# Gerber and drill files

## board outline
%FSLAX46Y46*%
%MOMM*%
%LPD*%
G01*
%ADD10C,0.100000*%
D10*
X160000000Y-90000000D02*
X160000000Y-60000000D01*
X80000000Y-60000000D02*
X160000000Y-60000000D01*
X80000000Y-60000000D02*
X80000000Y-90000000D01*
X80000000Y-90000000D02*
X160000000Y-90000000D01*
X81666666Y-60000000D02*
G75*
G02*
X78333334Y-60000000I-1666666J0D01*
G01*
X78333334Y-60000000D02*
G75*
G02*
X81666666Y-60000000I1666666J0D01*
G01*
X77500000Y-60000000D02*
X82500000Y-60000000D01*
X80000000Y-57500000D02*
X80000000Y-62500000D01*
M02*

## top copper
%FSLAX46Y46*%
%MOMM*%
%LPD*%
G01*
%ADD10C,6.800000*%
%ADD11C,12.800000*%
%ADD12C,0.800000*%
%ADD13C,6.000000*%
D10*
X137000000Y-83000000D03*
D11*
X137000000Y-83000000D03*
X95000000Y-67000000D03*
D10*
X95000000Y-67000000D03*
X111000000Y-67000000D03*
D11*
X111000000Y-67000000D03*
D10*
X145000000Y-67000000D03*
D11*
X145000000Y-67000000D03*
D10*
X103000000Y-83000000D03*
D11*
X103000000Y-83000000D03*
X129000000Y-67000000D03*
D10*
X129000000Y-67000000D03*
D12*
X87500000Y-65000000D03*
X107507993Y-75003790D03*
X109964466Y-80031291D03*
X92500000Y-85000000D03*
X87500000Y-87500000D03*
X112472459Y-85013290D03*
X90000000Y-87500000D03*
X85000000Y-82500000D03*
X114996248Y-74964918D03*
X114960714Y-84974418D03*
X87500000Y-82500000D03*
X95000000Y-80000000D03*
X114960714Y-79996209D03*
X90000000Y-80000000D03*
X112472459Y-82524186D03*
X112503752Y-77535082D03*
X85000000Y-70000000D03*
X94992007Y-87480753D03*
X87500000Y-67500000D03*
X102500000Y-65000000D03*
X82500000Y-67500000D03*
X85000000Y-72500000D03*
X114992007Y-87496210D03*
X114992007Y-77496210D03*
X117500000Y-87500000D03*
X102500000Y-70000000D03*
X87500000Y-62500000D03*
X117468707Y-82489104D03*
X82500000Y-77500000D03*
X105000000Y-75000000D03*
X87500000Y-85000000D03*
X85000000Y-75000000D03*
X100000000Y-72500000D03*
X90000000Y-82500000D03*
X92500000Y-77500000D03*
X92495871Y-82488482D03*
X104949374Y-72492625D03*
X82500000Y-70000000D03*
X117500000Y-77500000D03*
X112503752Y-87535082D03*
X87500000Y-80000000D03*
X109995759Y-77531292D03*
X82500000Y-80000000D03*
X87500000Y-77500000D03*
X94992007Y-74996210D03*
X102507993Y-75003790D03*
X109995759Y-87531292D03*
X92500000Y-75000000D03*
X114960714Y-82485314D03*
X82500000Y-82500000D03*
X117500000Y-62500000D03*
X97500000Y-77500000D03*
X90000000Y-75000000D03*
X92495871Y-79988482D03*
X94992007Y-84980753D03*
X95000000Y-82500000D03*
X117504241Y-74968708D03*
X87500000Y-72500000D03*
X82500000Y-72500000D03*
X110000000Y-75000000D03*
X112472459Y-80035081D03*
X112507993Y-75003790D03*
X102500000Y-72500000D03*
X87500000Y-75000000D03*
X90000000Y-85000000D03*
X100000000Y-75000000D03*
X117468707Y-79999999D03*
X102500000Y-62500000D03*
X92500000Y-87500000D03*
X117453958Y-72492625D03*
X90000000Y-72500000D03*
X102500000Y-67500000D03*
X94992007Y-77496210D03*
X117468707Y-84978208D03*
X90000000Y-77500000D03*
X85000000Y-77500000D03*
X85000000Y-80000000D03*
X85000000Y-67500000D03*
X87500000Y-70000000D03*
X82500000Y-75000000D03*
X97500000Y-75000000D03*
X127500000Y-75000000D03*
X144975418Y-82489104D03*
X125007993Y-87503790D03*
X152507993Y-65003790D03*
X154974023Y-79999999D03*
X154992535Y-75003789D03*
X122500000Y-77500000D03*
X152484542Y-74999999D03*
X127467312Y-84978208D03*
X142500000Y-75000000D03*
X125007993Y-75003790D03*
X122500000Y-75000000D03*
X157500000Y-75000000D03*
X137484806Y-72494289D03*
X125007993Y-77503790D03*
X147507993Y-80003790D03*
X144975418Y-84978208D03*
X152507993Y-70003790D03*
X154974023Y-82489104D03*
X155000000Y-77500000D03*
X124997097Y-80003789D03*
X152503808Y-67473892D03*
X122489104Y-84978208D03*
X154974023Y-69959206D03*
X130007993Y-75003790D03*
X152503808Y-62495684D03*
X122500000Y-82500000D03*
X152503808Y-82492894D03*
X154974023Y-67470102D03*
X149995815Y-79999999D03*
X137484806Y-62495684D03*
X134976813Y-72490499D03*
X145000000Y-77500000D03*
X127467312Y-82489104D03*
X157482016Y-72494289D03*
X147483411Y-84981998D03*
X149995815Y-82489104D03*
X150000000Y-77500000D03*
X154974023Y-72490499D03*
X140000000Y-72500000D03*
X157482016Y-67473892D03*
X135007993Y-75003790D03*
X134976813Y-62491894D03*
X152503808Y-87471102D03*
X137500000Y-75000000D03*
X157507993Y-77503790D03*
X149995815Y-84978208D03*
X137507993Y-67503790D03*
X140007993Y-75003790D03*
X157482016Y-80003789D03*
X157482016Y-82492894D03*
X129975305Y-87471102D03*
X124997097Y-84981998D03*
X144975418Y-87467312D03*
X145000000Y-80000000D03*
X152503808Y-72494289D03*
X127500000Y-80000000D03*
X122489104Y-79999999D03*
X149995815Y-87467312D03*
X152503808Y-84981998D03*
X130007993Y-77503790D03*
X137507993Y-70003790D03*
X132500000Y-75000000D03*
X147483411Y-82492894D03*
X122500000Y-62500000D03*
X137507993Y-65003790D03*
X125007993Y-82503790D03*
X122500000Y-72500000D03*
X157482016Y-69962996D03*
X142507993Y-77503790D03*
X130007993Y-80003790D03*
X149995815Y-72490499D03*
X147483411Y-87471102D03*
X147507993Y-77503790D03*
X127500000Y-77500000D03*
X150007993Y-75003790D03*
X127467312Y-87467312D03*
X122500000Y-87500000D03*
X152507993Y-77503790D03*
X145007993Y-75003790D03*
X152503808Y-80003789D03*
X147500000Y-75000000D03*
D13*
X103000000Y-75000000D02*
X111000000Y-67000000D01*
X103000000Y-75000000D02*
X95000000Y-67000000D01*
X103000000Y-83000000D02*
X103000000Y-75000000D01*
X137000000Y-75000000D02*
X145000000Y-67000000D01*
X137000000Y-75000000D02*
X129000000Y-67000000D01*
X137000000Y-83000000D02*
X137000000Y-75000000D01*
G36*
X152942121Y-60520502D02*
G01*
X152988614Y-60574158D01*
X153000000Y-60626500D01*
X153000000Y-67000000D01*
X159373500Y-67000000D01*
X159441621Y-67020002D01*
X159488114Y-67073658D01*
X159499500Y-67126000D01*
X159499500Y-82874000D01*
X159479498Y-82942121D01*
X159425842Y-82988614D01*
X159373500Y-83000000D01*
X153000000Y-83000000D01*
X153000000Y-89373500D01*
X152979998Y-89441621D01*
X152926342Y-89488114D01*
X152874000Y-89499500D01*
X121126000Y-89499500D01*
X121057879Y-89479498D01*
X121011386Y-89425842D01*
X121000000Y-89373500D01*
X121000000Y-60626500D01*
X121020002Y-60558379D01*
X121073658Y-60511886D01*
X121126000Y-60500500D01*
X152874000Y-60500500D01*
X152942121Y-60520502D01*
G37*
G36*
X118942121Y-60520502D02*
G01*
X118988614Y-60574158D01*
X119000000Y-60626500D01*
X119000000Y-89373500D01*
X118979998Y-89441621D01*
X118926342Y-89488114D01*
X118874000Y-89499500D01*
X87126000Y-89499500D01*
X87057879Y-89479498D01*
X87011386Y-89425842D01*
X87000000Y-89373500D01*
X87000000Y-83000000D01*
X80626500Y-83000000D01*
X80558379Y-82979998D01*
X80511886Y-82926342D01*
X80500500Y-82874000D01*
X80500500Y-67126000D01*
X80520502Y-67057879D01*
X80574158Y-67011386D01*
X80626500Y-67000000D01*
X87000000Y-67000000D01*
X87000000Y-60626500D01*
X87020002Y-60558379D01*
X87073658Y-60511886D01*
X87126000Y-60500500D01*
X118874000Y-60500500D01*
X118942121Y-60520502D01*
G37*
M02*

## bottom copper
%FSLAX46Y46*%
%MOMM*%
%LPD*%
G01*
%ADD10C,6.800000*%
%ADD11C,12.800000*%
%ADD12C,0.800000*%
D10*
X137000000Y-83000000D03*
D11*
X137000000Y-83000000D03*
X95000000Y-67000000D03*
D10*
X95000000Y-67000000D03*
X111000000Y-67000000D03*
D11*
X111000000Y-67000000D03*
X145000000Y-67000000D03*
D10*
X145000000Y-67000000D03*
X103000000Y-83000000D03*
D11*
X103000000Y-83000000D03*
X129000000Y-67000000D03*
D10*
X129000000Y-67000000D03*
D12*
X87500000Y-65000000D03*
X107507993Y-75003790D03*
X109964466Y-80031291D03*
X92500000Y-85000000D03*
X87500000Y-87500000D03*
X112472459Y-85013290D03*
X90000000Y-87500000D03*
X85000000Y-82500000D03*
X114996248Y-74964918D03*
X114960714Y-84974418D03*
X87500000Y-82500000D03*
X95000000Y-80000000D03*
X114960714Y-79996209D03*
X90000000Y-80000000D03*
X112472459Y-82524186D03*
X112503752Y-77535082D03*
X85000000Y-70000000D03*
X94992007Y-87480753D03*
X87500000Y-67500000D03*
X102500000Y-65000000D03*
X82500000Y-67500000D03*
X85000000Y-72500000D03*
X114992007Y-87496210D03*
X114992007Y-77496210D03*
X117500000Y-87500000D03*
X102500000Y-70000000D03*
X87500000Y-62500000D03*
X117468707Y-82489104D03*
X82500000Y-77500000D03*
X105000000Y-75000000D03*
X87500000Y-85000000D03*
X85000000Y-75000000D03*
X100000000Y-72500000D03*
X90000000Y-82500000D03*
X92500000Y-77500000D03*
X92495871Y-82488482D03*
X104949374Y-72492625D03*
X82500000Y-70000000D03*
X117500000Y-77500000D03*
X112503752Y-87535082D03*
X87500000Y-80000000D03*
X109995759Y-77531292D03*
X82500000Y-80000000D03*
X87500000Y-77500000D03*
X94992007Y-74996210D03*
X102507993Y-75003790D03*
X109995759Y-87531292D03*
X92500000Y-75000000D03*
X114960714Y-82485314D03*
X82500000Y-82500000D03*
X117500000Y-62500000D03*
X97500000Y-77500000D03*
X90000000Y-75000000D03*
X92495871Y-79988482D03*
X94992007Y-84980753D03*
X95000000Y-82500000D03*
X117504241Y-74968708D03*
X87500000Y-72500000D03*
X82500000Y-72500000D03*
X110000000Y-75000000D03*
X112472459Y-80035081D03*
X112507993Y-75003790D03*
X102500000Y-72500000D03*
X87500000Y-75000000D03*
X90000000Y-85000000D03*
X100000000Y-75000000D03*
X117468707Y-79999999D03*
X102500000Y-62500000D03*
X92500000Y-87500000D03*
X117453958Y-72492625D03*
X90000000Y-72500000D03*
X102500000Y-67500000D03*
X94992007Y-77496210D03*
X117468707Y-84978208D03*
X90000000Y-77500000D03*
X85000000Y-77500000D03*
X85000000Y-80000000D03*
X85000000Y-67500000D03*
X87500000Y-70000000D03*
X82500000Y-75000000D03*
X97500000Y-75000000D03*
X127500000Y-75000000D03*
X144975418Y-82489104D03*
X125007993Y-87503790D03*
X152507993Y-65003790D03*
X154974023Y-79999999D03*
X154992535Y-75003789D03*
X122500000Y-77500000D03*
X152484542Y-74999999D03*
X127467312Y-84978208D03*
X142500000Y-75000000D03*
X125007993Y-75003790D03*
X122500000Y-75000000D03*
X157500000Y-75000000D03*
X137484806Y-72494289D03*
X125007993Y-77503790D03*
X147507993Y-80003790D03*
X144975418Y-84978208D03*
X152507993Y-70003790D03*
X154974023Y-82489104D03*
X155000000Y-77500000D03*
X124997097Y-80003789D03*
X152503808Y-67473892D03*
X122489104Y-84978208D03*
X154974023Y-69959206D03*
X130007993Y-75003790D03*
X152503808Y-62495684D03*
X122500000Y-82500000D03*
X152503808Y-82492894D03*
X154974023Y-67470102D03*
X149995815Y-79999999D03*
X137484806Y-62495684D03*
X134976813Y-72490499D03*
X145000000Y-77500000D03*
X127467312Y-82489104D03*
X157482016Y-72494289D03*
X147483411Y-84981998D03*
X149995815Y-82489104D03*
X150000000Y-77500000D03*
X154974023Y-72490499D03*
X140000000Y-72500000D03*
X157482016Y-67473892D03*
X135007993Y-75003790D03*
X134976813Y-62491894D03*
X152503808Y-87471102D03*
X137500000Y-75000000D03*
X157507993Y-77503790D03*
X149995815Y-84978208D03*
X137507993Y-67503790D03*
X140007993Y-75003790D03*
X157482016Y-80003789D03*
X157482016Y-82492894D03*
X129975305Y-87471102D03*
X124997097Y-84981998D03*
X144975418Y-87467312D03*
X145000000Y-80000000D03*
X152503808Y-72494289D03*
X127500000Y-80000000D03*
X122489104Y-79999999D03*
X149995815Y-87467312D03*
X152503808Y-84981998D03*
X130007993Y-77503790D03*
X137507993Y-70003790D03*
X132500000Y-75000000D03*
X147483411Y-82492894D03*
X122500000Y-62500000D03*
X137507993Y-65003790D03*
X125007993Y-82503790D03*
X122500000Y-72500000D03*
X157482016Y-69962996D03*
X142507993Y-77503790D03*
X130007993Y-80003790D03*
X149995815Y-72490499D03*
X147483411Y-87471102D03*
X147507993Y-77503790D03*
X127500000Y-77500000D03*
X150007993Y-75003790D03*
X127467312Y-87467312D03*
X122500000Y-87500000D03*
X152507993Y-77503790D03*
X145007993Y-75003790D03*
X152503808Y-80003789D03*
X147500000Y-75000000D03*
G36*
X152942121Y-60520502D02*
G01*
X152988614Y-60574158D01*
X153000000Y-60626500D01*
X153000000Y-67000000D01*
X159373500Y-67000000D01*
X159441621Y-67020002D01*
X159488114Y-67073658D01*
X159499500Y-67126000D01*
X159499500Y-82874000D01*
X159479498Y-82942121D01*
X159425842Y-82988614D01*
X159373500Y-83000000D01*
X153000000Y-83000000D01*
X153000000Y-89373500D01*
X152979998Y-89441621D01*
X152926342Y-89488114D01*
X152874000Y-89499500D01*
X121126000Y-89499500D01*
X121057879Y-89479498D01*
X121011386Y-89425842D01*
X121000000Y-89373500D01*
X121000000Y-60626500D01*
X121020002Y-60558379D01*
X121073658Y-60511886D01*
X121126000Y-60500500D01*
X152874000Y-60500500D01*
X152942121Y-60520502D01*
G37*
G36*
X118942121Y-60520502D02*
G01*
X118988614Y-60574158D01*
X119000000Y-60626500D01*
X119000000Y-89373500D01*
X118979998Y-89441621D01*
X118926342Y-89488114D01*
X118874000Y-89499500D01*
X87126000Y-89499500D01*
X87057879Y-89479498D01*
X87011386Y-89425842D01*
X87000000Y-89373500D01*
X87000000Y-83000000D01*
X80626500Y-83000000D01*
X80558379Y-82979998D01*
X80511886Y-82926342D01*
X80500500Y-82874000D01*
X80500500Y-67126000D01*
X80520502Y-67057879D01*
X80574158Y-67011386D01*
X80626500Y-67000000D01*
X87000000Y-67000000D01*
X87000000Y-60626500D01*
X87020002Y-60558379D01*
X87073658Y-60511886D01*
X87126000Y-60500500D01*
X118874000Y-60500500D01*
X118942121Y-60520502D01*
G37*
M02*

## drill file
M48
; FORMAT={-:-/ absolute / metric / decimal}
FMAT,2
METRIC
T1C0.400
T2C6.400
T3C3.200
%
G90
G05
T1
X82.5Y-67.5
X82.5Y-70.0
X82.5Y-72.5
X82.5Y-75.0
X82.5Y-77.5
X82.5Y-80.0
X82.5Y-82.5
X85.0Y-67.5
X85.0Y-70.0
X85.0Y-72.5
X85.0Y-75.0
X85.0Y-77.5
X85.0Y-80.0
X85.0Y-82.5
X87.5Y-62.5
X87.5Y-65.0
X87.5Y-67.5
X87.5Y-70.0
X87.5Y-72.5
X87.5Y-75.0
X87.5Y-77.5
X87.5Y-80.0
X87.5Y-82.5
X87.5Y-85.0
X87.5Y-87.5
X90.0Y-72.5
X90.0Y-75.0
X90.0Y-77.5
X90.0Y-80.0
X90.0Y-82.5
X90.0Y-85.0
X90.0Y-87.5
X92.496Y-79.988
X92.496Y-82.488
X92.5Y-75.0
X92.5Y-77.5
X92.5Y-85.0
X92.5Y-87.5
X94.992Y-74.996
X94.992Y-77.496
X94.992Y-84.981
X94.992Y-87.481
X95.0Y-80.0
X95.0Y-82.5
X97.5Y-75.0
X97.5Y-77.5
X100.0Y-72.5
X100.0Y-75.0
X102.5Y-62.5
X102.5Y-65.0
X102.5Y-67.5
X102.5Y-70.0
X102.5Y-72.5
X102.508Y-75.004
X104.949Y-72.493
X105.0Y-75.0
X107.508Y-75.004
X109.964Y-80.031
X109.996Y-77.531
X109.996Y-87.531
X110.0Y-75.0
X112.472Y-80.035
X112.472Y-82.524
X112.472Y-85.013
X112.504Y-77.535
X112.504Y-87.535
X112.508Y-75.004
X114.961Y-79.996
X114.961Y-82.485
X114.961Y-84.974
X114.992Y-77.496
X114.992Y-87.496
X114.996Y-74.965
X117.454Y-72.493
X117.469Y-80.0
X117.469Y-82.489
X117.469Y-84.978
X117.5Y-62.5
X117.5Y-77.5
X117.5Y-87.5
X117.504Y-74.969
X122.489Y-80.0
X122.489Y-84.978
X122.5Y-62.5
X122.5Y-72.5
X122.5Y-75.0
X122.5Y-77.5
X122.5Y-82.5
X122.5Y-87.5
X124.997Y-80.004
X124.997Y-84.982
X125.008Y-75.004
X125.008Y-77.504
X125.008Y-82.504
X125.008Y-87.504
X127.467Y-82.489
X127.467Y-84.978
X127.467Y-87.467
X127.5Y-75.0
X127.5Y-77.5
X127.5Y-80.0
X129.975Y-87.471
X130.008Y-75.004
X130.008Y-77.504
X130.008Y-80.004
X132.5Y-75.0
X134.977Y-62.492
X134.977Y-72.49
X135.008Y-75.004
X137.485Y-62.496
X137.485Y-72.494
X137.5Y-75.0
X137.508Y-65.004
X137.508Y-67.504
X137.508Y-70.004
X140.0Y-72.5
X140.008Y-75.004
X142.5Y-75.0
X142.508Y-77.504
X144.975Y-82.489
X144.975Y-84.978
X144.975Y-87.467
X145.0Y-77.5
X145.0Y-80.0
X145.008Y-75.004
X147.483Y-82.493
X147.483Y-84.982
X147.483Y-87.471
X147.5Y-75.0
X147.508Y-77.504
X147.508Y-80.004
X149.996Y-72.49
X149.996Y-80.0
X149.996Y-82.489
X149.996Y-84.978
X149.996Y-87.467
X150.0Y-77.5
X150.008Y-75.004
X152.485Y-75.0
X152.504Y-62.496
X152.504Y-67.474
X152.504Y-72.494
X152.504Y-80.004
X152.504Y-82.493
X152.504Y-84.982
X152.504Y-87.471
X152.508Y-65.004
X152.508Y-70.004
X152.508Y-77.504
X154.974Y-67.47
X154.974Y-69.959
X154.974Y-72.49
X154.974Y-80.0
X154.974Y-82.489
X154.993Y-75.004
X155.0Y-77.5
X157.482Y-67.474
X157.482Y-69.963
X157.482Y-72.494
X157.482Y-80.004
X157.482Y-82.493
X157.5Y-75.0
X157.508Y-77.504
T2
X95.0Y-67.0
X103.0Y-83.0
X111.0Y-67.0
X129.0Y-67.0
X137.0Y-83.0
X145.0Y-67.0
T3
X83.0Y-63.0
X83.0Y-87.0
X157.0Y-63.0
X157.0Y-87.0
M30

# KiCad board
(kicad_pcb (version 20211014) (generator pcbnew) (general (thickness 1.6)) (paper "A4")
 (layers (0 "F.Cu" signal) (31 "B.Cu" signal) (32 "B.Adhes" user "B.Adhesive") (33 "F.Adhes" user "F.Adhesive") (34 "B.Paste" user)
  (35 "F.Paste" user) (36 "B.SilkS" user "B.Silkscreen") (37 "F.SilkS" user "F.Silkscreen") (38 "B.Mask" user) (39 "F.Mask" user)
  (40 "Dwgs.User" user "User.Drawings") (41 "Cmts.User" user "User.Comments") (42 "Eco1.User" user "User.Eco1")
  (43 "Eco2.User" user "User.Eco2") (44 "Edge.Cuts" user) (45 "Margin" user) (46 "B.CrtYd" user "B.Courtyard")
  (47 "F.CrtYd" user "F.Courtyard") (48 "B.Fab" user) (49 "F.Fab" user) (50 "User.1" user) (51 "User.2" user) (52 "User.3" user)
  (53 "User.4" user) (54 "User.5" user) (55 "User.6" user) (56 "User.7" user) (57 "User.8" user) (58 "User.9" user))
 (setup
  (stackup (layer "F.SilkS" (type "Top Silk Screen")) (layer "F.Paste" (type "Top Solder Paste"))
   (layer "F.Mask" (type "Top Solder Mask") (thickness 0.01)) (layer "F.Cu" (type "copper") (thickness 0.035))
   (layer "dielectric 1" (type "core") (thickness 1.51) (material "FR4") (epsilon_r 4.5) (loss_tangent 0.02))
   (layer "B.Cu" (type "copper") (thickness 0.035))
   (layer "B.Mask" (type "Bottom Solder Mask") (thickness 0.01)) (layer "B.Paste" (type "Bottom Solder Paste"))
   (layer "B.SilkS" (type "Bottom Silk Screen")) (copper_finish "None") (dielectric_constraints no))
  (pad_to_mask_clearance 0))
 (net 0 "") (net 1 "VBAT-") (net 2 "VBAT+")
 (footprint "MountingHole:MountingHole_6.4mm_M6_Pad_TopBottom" (layer "F.Cu") (at 137 83 90)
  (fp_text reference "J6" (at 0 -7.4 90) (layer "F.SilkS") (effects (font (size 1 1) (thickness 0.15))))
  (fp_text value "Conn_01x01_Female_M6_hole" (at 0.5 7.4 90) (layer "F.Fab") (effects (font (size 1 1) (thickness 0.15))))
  (pad "1" thru_hole circle locked (at 0 0 90) (size 6.8 6.8) (drill 6.4) (layers *.Cu *.Mask) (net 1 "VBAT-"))
  (pad "1" connect circle locked (at 0 0 90) (size 12.8 12.8) (layers "F.Cu" "F.Mask") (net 1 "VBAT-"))
  (pad "1" connect circle locked (at 0 0 90) (size 12.8 12.8) (layers "B.Cu" "B.Mask") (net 1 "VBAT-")))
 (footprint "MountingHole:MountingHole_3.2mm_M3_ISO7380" (layer "F.Cu") (at 157 87)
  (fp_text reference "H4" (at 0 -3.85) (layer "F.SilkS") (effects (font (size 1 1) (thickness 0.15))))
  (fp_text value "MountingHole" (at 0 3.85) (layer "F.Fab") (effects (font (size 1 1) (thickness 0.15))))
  (pad "" np_thru_hole circle locked (at 0 0) (size 3.2 3.2) (drill 3.2) (layers *.Cu *.Mask)))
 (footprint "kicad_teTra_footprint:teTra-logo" (layer "F.Cu") (at 86 75)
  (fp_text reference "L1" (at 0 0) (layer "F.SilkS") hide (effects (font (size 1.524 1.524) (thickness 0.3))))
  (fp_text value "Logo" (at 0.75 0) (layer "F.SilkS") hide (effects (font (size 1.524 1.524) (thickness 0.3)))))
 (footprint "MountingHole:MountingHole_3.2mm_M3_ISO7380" (layer "F.Cu") (at 83 87)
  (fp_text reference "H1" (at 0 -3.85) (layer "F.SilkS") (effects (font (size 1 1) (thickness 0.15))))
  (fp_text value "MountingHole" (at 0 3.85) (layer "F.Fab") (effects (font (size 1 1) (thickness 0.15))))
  (pad "" np_thru_hole circle locked (at 0 0) (size 3.2 3.2) (drill 3.2) (layers *.Cu *.Mask)))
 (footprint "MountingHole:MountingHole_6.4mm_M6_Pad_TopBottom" (layer "F.Cu") (at 95 67 90)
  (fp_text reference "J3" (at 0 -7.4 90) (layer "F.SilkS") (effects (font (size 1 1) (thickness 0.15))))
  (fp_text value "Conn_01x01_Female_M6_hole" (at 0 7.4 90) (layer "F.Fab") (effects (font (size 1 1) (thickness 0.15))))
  (pad "1" connect circle locked (at 0 0 90) (size 12.8 12.8) (layers "B.Cu" "B.Mask") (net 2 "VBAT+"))
  (pad "1" connect circle locked (at 0 0 90) (size 12.8 12.8) (layers "F.Cu" "F.Mask") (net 2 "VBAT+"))
  (pad "1" thru_hole circle locked (at 0 0 90) (size 6.8 6.8) (drill 6.4) (layers *.Cu *.Mask) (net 2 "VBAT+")))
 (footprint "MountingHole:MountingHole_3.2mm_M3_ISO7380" (layer "F.Cu") (at 83 63)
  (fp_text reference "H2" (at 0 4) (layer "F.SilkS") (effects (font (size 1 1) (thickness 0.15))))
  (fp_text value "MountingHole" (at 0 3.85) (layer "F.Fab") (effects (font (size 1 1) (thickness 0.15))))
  (pad "" np_thru_hole circle locked (at 0 0) (size 3.2 3.2) (drill 3.2) (layers *.Cu *.Mask)))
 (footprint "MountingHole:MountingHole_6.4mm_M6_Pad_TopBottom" (layer "F.Cu") (at 111 67 90)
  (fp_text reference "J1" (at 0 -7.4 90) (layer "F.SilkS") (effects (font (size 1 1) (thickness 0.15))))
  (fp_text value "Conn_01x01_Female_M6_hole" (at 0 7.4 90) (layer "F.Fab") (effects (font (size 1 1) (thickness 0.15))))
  (pad "1" thru_hole circle locked (at 0 0 90) (size 6.8 6.8) (drill 6.4) (layers *.Cu *.Mask) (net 2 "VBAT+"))
  (pad "1" connect circle locked (at 0 0 90) (size 12.8 12.8) (layers "F.Cu" "F.Mask") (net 2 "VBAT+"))
  (pad "1" connect circle locked (at 0 0 90) (size 12.8 12.8) (layers "B.Cu" "B.Mask") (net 2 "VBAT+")))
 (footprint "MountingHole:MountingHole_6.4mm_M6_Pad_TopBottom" (layer "F.Cu") (at 145 67 90)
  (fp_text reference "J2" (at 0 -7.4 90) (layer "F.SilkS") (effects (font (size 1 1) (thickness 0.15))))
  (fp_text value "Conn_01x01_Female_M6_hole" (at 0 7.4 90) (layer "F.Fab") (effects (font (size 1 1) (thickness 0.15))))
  (pad "1" connect circle locked (at 0 0 90) (size 12.8 12.8) (layers "B.Cu" "B.Mask") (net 1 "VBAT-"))
  (pad "1" thru_hole circle locked (at 0 0 90) (size 6.8 6.8) (drill 6.4) (layers *.Cu *.Mask) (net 1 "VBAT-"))
  (pad "1" connect circle locked (at 0 0 90) (size 12.8 12.8) (layers "F.Cu" "F.Mask") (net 1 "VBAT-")))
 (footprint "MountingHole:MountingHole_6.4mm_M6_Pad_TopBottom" (layer "F.Cu") (at 103 83 90)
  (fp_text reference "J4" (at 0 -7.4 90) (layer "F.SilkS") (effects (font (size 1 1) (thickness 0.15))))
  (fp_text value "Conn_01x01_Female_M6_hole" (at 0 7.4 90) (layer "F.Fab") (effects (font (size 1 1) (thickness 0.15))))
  (pad "1" thru_hole circle locked (at 0 0 90) (size 6.8 6.8) (drill 6.4) (layers *.Cu *.Mask) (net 2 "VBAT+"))
  (pad "1" connect circle locked (at 0 0 90) (size 12.8 12.8) (layers "B.Cu" "B.Mask") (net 2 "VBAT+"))
  (pad "1" connect circle locked (at 0 0 90) (size 12.8 12.8) (layers "F.Cu" "F.Mask") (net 2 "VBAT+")))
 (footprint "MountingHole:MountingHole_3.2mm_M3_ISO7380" (layer "F.Cu") (at 157 63)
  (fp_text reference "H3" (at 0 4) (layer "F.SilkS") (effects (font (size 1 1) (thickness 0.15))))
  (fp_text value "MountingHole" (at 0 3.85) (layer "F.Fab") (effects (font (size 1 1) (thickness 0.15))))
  (pad "" np_thru_hole circle locked (at 0 0) (size 3.2 3.2) (drill 3.2) (layers *.Cu *.Mask)))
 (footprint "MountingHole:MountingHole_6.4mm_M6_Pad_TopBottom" (layer "F.Cu") (at 129 67 90)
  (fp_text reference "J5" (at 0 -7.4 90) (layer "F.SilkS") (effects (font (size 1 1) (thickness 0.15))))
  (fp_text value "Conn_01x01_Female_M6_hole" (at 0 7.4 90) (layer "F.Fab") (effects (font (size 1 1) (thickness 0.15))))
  (pad "1" connect circle locked (at 0 0 90) (size 12.8 12.8) (layers "F.Cu" "F.Mask") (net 1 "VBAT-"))
  (pad "1" connect circle locked (at 0 0 90) (size 12.8 12.8) (layers "B.Cu" "B.Mask") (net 1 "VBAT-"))
  (pad "1" thru_hole circle locked (at 0 0 90) (size 6.8 6.8) (drill 6.4) (layers *.Cu *.Mask) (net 1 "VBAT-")))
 (gr_line (start 160 90) (end 160 60) (layer "Edge.Cuts") (width 0.1))
 (gr_line (start 80 60) (end 160 60) (layer "Edge.Cuts") (width 0.1))
 (gr_line (start 80 60) (end 80 90) (layer "Edge.Cuts") (width 0.1))
 (gr_line (start 80 90) (end 160 90) (layer "Edge.Cuts") (width 0.1))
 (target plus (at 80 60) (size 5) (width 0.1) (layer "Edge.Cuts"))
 (segment (start 103 75) (end 111 67) (width 6) (layer "F.Cu") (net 2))
 (segment (start 103 75) (end 95 67) (width 6) (layer "F.Cu") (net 2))
 (segment (start 103 83) (end 103 75) (width 6) (layer "F.Cu") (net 2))
 (via (at 87.5 65) (size 0.8) (drill 0.4) (layers "F.Cu" "B.Cu") (free) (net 2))
 (via (at 107.507993 75.00379) (size 0.8) (drill 0.4) (layers "F.Cu" "B.Cu") (free) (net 2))
 (via (at 109.964466 80.031291) (size 0.8) (drill 0.4) (layers "F.Cu" "B.Cu") (free) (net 2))
 (via (at 92.5 85) (size 0.8) (drill 0.4) (layers "F.Cu" "B.Cu") (free) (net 2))
 (via (at 87.5 87.5) (size 0.8) (drill 0.4) (layers "F.Cu" "B.Cu") (free) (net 2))
 (via (at 112.472459 85.01329) (size 0.8) (drill 0.4) (layers "F.Cu" "B.Cu") (free) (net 2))
 (via (at 90 87.5) (size 0.8) (drill 0.4) (layers "F.Cu" "B.Cu") (free) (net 2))
 (via (at 85 82.5) (size 0.8) (drill 0.4) (layers "F.Cu" "B.Cu") (free) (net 2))
 (via (at 114.996248 74.964918) (size 0.8) (drill 0.4) (layers "F.Cu" "B.Cu") (free) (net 2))
 (via (at 114.960714 84.974418) (size 0.8) (drill 0.4) (layers "F.Cu" "B.Cu") (free) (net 2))
 (via (at 87.5 82.5) (size 0.8) (drill 0.4) (layers "F.Cu" "B.Cu") (free) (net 2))
 (via (at 95 80) (size 0.8) (drill 0.4) (layers "F.Cu" "B.Cu") (free) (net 2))
 (via (at 114.960714 79.996209) (size 0.8) (drill 0.4) (layers "F.Cu" "B.Cu") (free) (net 2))
 (via (at 90 80) (size 0.8) (drill 0.4) (layers "F.Cu" "B.Cu") (free) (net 2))
 (via (at 112.472459 82.524186) (size 0.8) (drill 0.4) (layers "F.Cu" "B.Cu") (free) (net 2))
 (via (at 112.503752 77.535082) (size 0.8) (drill 0.4) (layers "F.Cu" "B.Cu") (free) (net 2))
 (via (at 85 70) (size 0.8) (drill 0.4) (layers "F.Cu" "B.Cu") (free) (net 2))
 (via (at 94.992007 87.480753) (size 0.8) (drill 0.4) (layers "F.Cu" "B.Cu") (free) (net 2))
 (via (at 87.5 67.5) (size 0.8) (drill 0.4) (layers "F.Cu" "B.Cu") (free) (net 2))
 (via (at 102.5 65) (size 0.8) (drill 0.4) (layers "F.Cu" "B.Cu") (free) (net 2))
 (via (at 82.5 67.5) (size 0.8) (drill 0.4) (layers "F.Cu" "B.Cu") (free) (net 2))
 (via (at 85 72.5) (size 0.8) (drill 0.4) (layers "F.Cu" "B.Cu") (free) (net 2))
 (via (at 114.992007 87.49621) (size 0.8) (drill 0.4) (layers "F.Cu" "B.Cu") (free) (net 2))
 (via (at 114.992007 77.49621) (size 0.8) (drill 0.4) (layers "F.Cu" "B.Cu") (free) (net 2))
 (via (at 117.5 87.5) (size 0.8) (drill 0.4) (layers "F.Cu" "B.Cu") (free) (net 2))
 (via (at 102.5 70) (size 0.8) (drill 0.4) (layers "F.Cu" "B.Cu") (free) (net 2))
 (via (at 87.5 62.5) (size 0.8) (drill 0.4) (layers "F.Cu" "B.Cu") (free) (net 2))
 (via (at 117.468707 82.489104) (size 0.8) (drill 0.4) (layers "F.Cu" "B.Cu") (free) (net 2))
 (via (at 82.5 77.5) (size 0.8) (drill 0.4) (layers "F.Cu" "B.Cu") (free) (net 2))
 (via (at 105 75) (size 0.8) (drill 0.4) (layers "F.Cu" "B.Cu") (free) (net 2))
 (via (at 87.5 85) (size 0.8) (drill 0.4) (layers "F.Cu" "B.Cu") (free) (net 2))
 (via (at 85 75) (size 0.8) (drill 0.4) (layers "F.Cu" "B.Cu") (free) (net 2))
 (via (at 100 72.5) (size 0.8) (drill 0.4) (layers "F.Cu" "B.Cu") (free) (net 2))
 (via (at 90 82.5) (size 0.8) (drill 0.4) (layers "F.Cu" "B.Cu") (free) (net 2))
 (via (at 92.5 77.5) (size 0.8) (drill 0.4) (layers "F.Cu" "B.Cu") (free) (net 2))
 (via (at 92.495871 82.488482) (size 0.8) (drill 0.4) (layers "F.Cu" "B.Cu") (free) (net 2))
 (via (at 104.949374 72.492625) (size 0.8) (drill 0.4) (layers "F.Cu" "B.Cu") (free) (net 2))
 (via (at 82.5 70) (size 0.8) (drill 0.4) (layers "F.Cu" "B.Cu") (free) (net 2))
 (via (at 117.5 77.5) (size 0.8) (drill 0.4) (layers "F.Cu" "B.Cu") (free) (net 2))
 (via (at 112.503752 87.535082) (size 0.8) (drill 0.4) (layers "F.Cu" "B.Cu") (free) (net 2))
 (via (at 87.5 80) (size 0.8) (drill 0.4) (layers "F.Cu" "B.Cu") (free) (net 2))
 (via (at 109.995759 77.531292) (size 0.8) (drill 0.4) (layers "F.Cu" "B.Cu") (free) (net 2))
 (via (at 82.5 80) (size 0.8) (drill 0.4) (layers "F.Cu" "B.Cu") (free) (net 2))
 (via (at 87.5 77.5) (size 0.8) (drill 0.4) (layers "F.Cu" "B.Cu") (free) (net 2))
 (via (at 94.992007 74.99621) (size 0.8) (drill 0.4) (layers "F.Cu" "B.Cu") (free) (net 2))
 (via (at 102.507993 75.00379) (size 0.8) (drill 0.4) (layers "F.Cu" "B.Cu") (free) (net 2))
 (via (at 109.995759 87.531292) (size 0.8) (drill 0.4) (layers "F.Cu" "B.Cu") (free) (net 2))
 (via (at 92.5 75) (size 0.8) (drill 0.4) (layers "F.Cu" "B.Cu") (free) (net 2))
 (via (at 114.960714 82.485314) (size 0.8) (drill 0.4) (layers "F.Cu" "B.Cu") (free) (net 2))
 (via (at 82.5 82.5) (size 0.8) (drill 0.4) (layers "F.Cu" "B.Cu") (free) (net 2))
 (via (at 117.5 62.5) (size 0.8) (drill 0.4) (layers "F.Cu" "B.Cu") (free) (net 2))
 (via (at 97.5 77.5) (size 0.8) (drill 0.4) (layers "F.Cu" "B.Cu") (free) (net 2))
 (via (at 90 75) (size 0.8) (drill 0.4) (layers "F.Cu" "B.Cu") (free) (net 2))
 (via (at 92.495871 79.988482) (size 0.8) (drill 0.4) (layers "F.Cu" "B.Cu") (free) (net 2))
 (via (at 94.992007 84.980753) (size 0.8) (drill 0.4) (layers "F.Cu" "B.Cu") (free) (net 2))
 (via (at 95 82.5) (size 0.8) (drill 0.4) (layers "F.Cu" "B.Cu") (free) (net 2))
 (via (at 117.504241 74.968708) (size 0.8) (drill 0.4) (layers "F.Cu" "B.Cu") (free) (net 2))
 (via (at 87.5 72.5) (size 0.8) (drill 0.4) (layers "F.Cu" "B.Cu") (free) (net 2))
 (via (at 82.5 72.5) (size 0.8) (drill 0.4) (layers "F.Cu" "B.Cu") (free) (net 2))
 (via (at 110 75) (size 0.8) (drill 0.4) (layers "F.Cu" "B.Cu") (free) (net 2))
 (via (at 112.472459 80.035081) (size 0.8) (drill 0.4) (layers "F.Cu" "B.Cu") (free) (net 2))
 (via (at 112.507993 75.00379) (size 0.8) (drill 0.4) (layers "F.Cu" "B.Cu") (free) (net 2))
 (via (at 102.5 72.5) (size 0.8) (drill 0.4) (layers "F.Cu" "B.Cu") (free) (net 2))
 (via (at 87.5 75) (size 0.8) (drill 0.4) (layers "F.Cu" "B.Cu") (free) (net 2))
 (via (at 90 85) (size 0.8) (drill 0.4) (layers "F.Cu" "B.Cu") (free) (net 2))
 (via (at 100 75) (size 0.8) (drill 0.4) (layers "F.Cu" "B.Cu") (free) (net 2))
 (via (at 117.468707 79.999999) (size 0.8) (drill 0.4) (layers "F.Cu" "B.Cu") (free) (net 2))
 (via (at 102.5 62.5) (size 0.8) (drill 0.4) (layers "F.Cu" "B.Cu") (free) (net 2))
 (via (at 92.5 87.5) (size 0.8) (drill 0.4) (layers "F.Cu" "B.Cu") (free) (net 2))
 (via (at 117.453958 72.492625) (size 0.8) (drill 0.4) (layers "F.Cu" "B.Cu") (free) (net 2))
 (via (at 90 72.5) (size 0.8) (drill 0.4) (layers "F.Cu" "B.Cu") (free) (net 2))
 (via (at 102.5 67.5) (size 0.8) (drill 0.4) (layers "F.Cu" "B.Cu") (free) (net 2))
 (via (at 94.992007 77.49621) (size 0.8) (drill 0.4) (layers "F.Cu" "B.Cu") (free) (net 2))
 (via (at 117.468707 84.978208) (size 0.8) (drill 0.4) (layers "F.Cu" "B.Cu") (free) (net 2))
 (via (at 90 77.5) (size 0.8) (drill 0.4) (layers "F.Cu" "B.Cu") (free) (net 2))
 (via (at 85 77.5) (size 0.8) (drill 0.4) (layers "F.Cu" "B.Cu") (free) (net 2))
 (via (at 85 80) (size 0.8) (drill 0.4) (layers "F.Cu" "B.Cu") (free) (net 2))
 (via (at 85 67.5) (size 0.8) (drill 0.4) (layers "F.Cu" "B.Cu") (free) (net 2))
 (via (at 87.5 70) (size 0.8) (drill 0.4) (layers "F.Cu" "B.Cu") (free) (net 2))
 (via (at 82.5 75) (size 0.8) (drill 0.4) (layers "F.Cu" "B.Cu") (free) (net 2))
 (via (at 97.5 75) (size 0.8) (drill 0.4) (layers "F.Cu" "B.Cu") (free) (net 2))
 (segment (start 137 75) (end 145 67) (width 6) (layer "F.Cu") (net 1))
 (segment (start 137 75) (end 129 67) (width 6) (layer "F.Cu") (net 1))
 (segment (start 137 83) (end 137 75) (width 6) (layer "F.Cu") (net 1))
 (via (at 127.5 75) (size 0.8) (drill 0.4) (layers "F.Cu" "B.Cu") (free) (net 1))
 (via (at 144.975418 82.489104) (size 0.8) (drill 0.4) (layers "F.Cu" "B.Cu") (free) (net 1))
 (via (at 125.007993 87.50379) (size 0.8) (drill 0.4) (layers "F.Cu" "B.Cu") (free) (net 1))
 (via (at 152.507993 65.00379) (size 0.8) (drill 0.4) (layers "F.Cu" "B.Cu") (free) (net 1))
 (via (at 154.974023 79.999999) (size 0.8) (drill 0.4) (layers "F.Cu" "B.Cu") (free) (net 1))
 (via (at 154.992535 75.003789) (size 0.8) (drill 0.4) (layers "F.Cu" "B.Cu") (free) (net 1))
 (via (at 122.5 77.5) (size 0.8) (drill 0.4) (layers "F.Cu" "B.Cu") (free) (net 1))
 (via (at 152.484542 74.999999) (size 0.8) (drill 0.4) (layers "F.Cu" "B.Cu") (free) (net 1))
 (via (at 127.467312 84.978208) (size 0.8) (drill 0.4) (layers "F.Cu" "B.Cu") (free) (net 1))
 (via (at 142.5 75) (size 0.8) (drill 0.4) (layers "F.Cu" "B.Cu") (free) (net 1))
 (via (at 125.007993 75.00379) (size 0.8) (drill 0.4) (layers "F.Cu" "B.Cu") (free) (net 1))
 (via (at 122.5 75) (size 0.8) (drill 0.4) (layers "F.Cu" "B.Cu") (free) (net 1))
 (via (at 157.5 75) (size 0.8) (drill 0.4) (layers "F.Cu" "B.Cu") (free) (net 1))
 (via (at 137.484806 72.494289) (size 0.8) (drill 0.4) (layers "F.Cu" "B.Cu") (free) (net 1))
 (via (at 125.007993 77.50379) (size 0.8) (drill 0.4) (layers "F.Cu" "B.Cu") (free) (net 1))
 (via (at 147.507993 80.00379) (size 0.8) (drill 0.4) (layers "F.Cu" "B.Cu") (free) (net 1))
 (via (at 144.975418 84.978208) (size 0.8) (drill 0.4) (layers "F.Cu" "B.Cu") (free) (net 1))
 (via (at 152.507993 70.00379) (size 0.8) (drill 0.4) (layers "F.Cu" "B.Cu") (free) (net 1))
 (via (at 154.974023 82.489104) (size 0.8) (drill 0.4) (layers "F.Cu" "B.Cu") (free) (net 1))
 (via (at 155 77.5) (size 0.8) (drill 0.4) (layers "F.Cu" "B.Cu") (free) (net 1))
 (via (at 124.997097 80.003789) (size 0.8) (drill 0.4) (layers "F.Cu" "B.Cu") (free) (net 1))
 (via (at 152.503808 67.473892) (size 0.8) (drill 0.4) (layers "F.Cu" "B.Cu") (free) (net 1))
 (via (at 122.489104 84.978208) (size 0.8) (drill 0.4) (layers "F.Cu" "B.Cu") (free) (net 1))
 (via (at 154.974023 69.959206) (size 0.8) (drill 0.4) (layers "F.Cu" "B.Cu") (free) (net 1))
 (via (at 130.007993 75.00379) (size 0.8) (drill 0.4) (layers "F.Cu" "B.Cu") (free) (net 1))
 (via (at 152.503808 62.495684) (size 0.8) (drill 0.4) (layers "F.Cu" "B.Cu") (free) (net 1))
 (via (at 122.5 82.5) (size 0.8) (drill 0.4) (layers "F.Cu" "B.Cu") (free) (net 1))
 (via (at 152.503808 82.492894) (size 0.8) (drill 0.4) (layers "F.Cu" "B.Cu") (free) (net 1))
 (via (at 154.974023 67.470102) (size 0.8) (drill 0.4) (layers "F.Cu" "B.Cu") (free) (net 1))
 (via (at 149.995815 79.999999) (size 0.8) (drill 0.4) (layers "F.Cu" "B.Cu") (free) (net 1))
 (via (at 137.484806 62.495684) (size 0.8) (drill 0.4) (layers "F.Cu" "B.Cu") (free) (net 1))
 (via (at 134.976813 72.490499) (size 0.8) (drill 0.4) (layers "F.Cu" "B.Cu") (free) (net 1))
 (via (at 145 77.5) (size 0.8) (drill 0.4) (layers "F.Cu" "B.Cu") (free) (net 1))
 (via (at 127.467312 82.489104) (size 0.8) (drill 0.4) (layers "F.Cu" "B.Cu") (free) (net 1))
 (via (at 157.482016 72.494289) (size 0.8) (drill 0.4) (layers "F.Cu" "B.Cu") (free) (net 1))
 (via (at 147.483411 84.981998) (size 0.8) (drill 0.4) (layers "F.Cu" "B.Cu") (free) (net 1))
 (via (at 149.995815 82.489104) (size 0.8) (drill 0.4) (layers "F.Cu" "B.Cu") (free) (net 1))
 (via (at 150 77.5) (size 0.8) (drill 0.4) (layers "F.Cu" "B.Cu") (free) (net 1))
 (via (at 154.974023 72.490499) (size 0.8) (drill 0.4) (layers "F.Cu" "B.Cu") (free) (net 1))
 (via (at 140 72.5) (size 0.8) (drill 0.4) (layers "F.Cu" "B.Cu") (free) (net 1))
 (via (at 157.482016 67.473892) (size 0.8) (drill 0.4) (layers "F.Cu" "B.Cu") (free) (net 1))
 (via (at 135.007993 75.00379) (size 0.8) (drill 0.4) (layers "F.Cu" "B.Cu") (free) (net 1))
 (via (at 134.976813 62.491894) (size 0.8) (drill 0.4) (layers "F.Cu" "B.Cu") (free) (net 1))
 (via (at 152.503808 87.471102) (size 0.8) (drill 0.4) (layers "F.Cu" "B.Cu") (free) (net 1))
 (via (at 137.5 75) (size 0.8) (drill 0.4) (layers "F.Cu" "B.Cu") (free) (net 1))
 (via (at 157.507993 77.50379) (size 0.8) (drill 0.4) (layers "F.Cu" "B.Cu") (free) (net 1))
 (via (at 149.995815 84.978208) (size 0.8) (drill 0.4) (layers "F.Cu" "B.Cu") (free) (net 1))
 (via (at 137.507993 67.50379) (size 0.8) (drill 0.4) (layers "F.Cu" "B.Cu") (free) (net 1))
 (via (at 140.007993 75.00379) (size 0.8) (drill 0.4) (layers "F.Cu" "B.Cu") (free) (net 1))
 (via (at 157.482016 80.003789) (size 0.8) (drill 0.4) (layers "F.Cu" "B.Cu") (free) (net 1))
 (via (at 157.482016 82.492894) (size 0.8) (drill 0.4) (layers "F.Cu" "B.Cu") (free) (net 1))
 (via (at 129.975305 87.471102) (size 0.8) (drill 0.4) (layers "F.Cu" "B.Cu") (free) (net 1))
 (via (at 124.997097 84.981998) (size 0.8) (drill 0.4) (layers "F.Cu" "B.Cu") (free) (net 1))
 (via (at 144.975418 87.467312) (size 0.8) (drill 0.4) (layers "F.Cu" "B.Cu") (free) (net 1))
 (via (at 145 80) (size 0.8) (drill 0.4) (layers "F.Cu" "B.Cu") (free) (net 1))
 (via (at 152.503808 72.494289) (size 0.8) (drill 0.4) (layers "F.Cu" "B.Cu") (free) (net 1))
 (via (at 127.5 80) (size 0.8) (drill 0.4) (layers "F.Cu" "B.Cu") (free) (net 1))
 (via (at 122.489104 79.999999) (size 0.8) (drill 0.4) (layers "F.Cu" "B.Cu") (free) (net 1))
 (via (at 149.995815 87.467312) (size 0.8) (drill 0.4) (layers "F.Cu" "B.Cu") (free) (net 1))
 (via (at 152.503808 84.981998) (size 0.8) (drill 0.4) (layers "F.Cu" "B.Cu") (free) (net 1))
 (via (at 130.007993 77.50379) (size 0.8) (drill 0.4) (layers "F.Cu" "B.Cu") (free) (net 1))
 (via (at 137.507993 70.00379) (size 0.8) (drill 0.4) (layers "F.Cu" "B.Cu") (free) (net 1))
 (via (at 132.5 75) (size 0.8) (drill 0.4) (layers "F.Cu" "B.Cu") (free) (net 1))
 (via (at 147.483411 82.492894) (size 0.8) (drill 0.4) (layers "F.Cu" "B.Cu") (free) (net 1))
 (via (at 122.5 62.5) (size 0.8) (drill 0.4) (layers "F.Cu" "B.Cu") (free) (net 1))
 (via (at 137.507993 65.00379) (size 0.8) (drill 0.4) (layers "F.Cu" "B.Cu") (free) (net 1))
 (via (at 125.007993 82.50379) (size 0.8) (drill 0.4) (layers "F.Cu" "B.Cu") (free) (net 1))
 (via (at 122.5 72.5) (size 0.8) (drill 0.4) (layers "F.Cu" "B.Cu") (free) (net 1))
 (via (at 157.482016 69.962996) (size 0.8) (drill 0.4) (layers "F.Cu" "B.Cu") (free) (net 1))
 (via (at 142.507993 77.50379) (size 0.8) (drill 0.4) (layers "F.Cu" "B.Cu") (free) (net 1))
 (via (at 130.007993 80.00379) (size 0.8) (drill 0.4) (layers "F.Cu" "B.Cu") (free) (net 1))
 (via (at 149.995815 72.490499) (size 0.8) (drill 0.4) (layers "F.Cu" "B.Cu") (free) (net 1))
 (via (at 147.483411 87.471102) (size 0.8) (drill 0.4) (layers "F.Cu" "B.Cu") (free) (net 1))
 (via (at 147.507993 77.50379) (size 0.8) (drill 0.4) (layers "F.Cu" "B.Cu") (free) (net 1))
 (via (at 127.5 77.5) (size 0.8) (drill 0.4) (layers "F.Cu" "B.Cu") (free) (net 1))
 (via (at 150.007993 75.00379) (size 0.8) (drill 0.4) (layers "F.Cu" "B.Cu") (free) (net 1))
 (via (at 127.467312 87.467312) (size 0.8) (drill 0.4) (layers "F.Cu" "B.Cu") (free) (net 1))
 (via (at 122.5 87.5) (size 0.8) (drill 0.4) (layers "F.Cu" "B.Cu") (free) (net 1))
 (via (at 152.507993 77.50379) (size 0.8) (drill 0.4) (layers "F.Cu" "B.Cu") (free) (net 1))
 (via (at 145.007993 75.00379) (size 0.8) (drill 0.4) (layers "F.Cu" "B.Cu") (free) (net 1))
 (via (at 152.503808 80.003789) (size 0.8) (drill 0.4) (layers "F.Cu" "B.Cu") (free) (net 1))
 (via (at 147.5 75) (size 0.8) (drill 0.4) (layers "F.Cu" "B.Cu") (free) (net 1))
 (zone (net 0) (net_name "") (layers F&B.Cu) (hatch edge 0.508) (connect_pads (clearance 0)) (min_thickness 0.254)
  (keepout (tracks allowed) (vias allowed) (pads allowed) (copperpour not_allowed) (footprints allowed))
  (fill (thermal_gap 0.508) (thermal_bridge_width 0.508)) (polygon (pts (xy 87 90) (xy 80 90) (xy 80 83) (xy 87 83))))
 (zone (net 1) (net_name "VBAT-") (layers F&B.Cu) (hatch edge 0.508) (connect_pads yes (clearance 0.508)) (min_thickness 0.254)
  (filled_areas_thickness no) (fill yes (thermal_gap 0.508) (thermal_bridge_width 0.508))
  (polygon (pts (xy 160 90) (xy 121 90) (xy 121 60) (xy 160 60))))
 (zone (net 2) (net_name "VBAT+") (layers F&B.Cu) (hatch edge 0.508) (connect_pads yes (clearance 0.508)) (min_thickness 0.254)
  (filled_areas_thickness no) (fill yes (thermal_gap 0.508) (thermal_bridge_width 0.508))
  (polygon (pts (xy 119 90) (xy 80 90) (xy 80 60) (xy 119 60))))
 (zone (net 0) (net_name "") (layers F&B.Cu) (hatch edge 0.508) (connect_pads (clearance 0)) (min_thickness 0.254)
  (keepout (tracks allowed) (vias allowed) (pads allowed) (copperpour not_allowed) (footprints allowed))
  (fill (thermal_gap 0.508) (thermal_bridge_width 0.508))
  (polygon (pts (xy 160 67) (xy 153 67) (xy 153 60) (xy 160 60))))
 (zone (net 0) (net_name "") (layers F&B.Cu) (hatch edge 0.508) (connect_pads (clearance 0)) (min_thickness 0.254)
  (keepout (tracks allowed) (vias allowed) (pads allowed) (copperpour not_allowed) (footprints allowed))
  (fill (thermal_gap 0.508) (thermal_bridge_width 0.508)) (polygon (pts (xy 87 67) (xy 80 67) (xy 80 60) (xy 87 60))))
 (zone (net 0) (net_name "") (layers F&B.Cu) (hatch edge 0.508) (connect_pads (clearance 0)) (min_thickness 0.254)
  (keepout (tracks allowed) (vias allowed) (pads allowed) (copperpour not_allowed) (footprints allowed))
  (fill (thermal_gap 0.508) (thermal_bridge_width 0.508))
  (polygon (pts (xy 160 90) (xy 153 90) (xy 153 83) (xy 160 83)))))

